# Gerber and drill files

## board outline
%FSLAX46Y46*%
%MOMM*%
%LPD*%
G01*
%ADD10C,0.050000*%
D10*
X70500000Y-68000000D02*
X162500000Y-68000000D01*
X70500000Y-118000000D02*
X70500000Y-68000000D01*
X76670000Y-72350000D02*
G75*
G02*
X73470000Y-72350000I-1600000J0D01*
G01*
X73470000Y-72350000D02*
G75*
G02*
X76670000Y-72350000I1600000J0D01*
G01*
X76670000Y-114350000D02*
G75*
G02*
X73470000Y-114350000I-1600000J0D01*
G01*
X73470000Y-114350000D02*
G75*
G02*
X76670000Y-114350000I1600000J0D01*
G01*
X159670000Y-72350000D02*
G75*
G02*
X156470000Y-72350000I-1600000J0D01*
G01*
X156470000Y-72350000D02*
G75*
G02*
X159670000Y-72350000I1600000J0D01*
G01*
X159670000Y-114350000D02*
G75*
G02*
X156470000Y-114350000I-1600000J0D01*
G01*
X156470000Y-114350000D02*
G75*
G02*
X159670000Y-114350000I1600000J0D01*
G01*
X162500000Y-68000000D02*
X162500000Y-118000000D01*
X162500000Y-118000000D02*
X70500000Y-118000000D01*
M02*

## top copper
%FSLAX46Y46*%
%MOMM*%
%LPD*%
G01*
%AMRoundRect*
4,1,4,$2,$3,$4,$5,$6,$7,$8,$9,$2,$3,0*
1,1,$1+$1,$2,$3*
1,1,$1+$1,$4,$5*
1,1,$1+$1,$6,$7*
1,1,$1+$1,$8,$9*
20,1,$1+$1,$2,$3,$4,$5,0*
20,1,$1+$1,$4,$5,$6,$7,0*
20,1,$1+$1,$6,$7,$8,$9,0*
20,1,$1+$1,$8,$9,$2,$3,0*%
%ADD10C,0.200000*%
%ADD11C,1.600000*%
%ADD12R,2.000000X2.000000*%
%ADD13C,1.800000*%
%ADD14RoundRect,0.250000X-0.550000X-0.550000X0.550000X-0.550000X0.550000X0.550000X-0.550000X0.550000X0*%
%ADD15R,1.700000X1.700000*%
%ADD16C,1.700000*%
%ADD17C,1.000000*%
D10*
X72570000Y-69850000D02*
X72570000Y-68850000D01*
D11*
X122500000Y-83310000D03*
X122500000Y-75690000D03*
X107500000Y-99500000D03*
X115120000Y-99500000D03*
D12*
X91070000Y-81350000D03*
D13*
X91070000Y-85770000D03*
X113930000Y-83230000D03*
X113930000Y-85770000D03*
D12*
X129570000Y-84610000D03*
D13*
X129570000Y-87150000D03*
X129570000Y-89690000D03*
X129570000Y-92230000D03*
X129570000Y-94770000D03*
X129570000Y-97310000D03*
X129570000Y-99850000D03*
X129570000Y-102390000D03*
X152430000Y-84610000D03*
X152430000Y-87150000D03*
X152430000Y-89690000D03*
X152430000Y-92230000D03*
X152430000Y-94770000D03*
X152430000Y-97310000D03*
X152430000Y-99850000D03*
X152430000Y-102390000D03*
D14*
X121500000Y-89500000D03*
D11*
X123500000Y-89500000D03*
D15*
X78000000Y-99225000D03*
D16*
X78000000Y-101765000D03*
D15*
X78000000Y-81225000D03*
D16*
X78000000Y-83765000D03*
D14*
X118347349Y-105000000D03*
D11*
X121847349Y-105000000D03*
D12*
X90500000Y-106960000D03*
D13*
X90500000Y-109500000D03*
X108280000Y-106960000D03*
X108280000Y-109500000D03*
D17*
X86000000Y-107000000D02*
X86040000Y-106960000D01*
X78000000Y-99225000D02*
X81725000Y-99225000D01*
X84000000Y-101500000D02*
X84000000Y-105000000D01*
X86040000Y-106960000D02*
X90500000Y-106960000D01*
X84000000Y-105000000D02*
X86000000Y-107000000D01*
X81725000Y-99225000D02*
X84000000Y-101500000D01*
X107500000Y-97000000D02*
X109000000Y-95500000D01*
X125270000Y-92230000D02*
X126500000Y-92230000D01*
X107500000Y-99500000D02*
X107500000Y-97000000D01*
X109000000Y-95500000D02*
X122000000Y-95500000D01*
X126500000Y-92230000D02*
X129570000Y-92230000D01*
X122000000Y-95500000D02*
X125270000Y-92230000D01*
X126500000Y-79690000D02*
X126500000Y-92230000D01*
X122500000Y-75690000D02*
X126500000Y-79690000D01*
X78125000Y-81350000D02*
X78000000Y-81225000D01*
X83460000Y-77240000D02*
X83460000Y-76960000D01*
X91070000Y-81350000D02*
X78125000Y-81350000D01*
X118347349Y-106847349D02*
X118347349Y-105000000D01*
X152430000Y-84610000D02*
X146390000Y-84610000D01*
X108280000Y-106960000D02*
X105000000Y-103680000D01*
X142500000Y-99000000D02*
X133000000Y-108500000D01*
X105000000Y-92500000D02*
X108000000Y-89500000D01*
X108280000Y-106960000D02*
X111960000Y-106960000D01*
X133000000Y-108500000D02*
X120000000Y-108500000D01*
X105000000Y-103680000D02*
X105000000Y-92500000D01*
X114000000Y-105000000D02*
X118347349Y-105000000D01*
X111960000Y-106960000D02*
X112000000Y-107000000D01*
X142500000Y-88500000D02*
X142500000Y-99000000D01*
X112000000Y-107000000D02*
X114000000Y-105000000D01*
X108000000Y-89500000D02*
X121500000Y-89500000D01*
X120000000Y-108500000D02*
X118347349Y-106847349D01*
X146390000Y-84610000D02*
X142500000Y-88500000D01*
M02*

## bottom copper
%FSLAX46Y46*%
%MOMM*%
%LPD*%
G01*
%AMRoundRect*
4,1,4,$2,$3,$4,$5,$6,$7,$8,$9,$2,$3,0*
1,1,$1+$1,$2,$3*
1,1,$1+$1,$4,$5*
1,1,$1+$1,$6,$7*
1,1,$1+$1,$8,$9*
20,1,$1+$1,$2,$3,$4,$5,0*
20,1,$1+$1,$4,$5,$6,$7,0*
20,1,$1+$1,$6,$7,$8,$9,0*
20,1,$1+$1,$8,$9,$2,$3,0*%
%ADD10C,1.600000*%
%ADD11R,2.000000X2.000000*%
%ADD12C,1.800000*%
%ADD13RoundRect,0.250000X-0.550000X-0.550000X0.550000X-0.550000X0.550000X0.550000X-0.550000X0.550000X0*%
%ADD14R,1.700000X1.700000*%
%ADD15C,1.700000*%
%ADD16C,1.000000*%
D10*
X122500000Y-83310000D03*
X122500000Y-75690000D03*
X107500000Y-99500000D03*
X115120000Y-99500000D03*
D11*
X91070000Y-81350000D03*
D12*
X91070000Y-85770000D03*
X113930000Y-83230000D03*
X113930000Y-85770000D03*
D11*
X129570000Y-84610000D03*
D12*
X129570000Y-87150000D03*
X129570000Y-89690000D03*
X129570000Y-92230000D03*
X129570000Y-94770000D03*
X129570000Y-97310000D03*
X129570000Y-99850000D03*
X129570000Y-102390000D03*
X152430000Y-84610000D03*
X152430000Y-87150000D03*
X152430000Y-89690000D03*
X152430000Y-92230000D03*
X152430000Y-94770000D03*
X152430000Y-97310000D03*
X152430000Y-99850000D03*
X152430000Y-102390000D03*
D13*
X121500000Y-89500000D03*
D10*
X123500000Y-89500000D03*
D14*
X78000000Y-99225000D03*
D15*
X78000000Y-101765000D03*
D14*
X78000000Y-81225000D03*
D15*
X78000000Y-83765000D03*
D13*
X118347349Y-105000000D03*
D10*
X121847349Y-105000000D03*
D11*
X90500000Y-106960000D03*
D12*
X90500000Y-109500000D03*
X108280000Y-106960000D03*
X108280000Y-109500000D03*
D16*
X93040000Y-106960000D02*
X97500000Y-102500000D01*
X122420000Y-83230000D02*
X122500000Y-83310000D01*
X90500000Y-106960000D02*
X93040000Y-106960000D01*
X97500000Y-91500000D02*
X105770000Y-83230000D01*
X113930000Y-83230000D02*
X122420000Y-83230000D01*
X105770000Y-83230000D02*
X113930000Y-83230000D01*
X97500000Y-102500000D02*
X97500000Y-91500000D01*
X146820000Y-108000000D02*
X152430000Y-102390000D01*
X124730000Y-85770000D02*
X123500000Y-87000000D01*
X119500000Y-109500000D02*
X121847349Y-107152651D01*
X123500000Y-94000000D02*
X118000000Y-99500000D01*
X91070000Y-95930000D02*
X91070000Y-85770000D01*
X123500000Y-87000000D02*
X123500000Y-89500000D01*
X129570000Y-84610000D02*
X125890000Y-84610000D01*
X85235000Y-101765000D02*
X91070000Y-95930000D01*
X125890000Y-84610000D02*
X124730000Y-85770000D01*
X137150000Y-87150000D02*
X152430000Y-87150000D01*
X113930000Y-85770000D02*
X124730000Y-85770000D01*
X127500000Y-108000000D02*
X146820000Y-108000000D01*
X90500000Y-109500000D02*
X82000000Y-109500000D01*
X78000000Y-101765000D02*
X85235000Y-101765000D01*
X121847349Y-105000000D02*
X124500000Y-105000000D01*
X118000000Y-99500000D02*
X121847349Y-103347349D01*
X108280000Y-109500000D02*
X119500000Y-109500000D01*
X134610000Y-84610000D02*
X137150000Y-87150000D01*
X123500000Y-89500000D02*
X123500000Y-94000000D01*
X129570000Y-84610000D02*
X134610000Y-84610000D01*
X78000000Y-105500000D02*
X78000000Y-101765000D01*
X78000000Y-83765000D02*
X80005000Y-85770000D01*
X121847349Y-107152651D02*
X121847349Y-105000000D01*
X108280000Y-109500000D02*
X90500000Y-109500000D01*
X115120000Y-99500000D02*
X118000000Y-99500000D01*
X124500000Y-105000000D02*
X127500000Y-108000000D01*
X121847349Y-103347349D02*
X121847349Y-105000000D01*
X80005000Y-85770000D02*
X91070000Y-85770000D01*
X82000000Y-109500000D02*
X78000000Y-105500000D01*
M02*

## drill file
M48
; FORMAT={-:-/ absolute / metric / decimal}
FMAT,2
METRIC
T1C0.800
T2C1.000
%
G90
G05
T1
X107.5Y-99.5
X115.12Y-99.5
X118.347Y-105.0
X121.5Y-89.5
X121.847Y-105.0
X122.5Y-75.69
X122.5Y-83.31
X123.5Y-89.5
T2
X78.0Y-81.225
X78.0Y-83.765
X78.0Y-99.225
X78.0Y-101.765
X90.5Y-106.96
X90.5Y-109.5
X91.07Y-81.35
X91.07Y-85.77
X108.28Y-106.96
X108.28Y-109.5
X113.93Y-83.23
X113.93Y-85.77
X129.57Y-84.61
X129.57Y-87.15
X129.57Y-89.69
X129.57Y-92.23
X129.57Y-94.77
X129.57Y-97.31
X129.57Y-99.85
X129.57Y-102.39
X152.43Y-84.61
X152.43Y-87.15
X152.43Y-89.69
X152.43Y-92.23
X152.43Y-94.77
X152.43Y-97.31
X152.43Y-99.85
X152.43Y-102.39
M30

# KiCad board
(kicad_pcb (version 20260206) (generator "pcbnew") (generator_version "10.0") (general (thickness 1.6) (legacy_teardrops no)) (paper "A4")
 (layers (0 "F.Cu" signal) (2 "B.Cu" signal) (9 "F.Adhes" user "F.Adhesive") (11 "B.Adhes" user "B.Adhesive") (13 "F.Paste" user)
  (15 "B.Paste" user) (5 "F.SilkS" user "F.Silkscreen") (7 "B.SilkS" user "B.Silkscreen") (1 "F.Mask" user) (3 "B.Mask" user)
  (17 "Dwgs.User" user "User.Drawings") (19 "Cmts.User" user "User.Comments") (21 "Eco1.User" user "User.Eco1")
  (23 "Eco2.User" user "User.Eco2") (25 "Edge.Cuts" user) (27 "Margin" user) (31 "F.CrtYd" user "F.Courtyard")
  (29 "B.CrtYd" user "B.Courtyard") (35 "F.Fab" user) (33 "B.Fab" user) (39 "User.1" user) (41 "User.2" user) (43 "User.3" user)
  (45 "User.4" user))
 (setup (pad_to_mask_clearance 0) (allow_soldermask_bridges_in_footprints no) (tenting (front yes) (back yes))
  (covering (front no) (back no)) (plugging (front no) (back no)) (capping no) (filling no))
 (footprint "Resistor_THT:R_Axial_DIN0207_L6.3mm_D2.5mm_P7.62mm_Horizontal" (layer "F.Cu") (at 122.5 83.31 90)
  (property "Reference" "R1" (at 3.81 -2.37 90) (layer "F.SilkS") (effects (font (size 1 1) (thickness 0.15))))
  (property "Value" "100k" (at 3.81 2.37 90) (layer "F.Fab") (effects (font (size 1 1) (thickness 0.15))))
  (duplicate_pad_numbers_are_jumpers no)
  (pad "1" thru_hole circle (at 0 0 90) (size 1.6 1.6) (drill 0.8) (layers "*.Cu" "*.Mask") (remove_unused_layers no) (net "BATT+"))
  (pad "2" thru_hole circle (at 7.62 0 90) (size 1.6 1.6) (drill 0.8) (layers "*.Cu" "*.Mask") (remove_unused_layers no) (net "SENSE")))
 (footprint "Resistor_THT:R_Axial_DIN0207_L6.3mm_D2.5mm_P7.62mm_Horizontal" (layer "F.Cu") (at 107.5 99.5)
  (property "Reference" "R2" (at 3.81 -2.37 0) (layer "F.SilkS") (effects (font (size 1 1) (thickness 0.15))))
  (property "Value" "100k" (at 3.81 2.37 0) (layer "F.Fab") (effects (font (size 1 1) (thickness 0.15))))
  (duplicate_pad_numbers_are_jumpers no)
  (pad "1" thru_hole circle (at 0 0) (size 1.6 1.6) (drill 0.8) (layers "*.Cu" "*.Mask") (remove_unused_layers no) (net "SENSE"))
  (pad "2" thru_hole circle (at 7.62 0) (size 1.6 1.6) (drill 0.8) (layers "*.Cu" "*.Mask") (remove_unused_layers no) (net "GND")))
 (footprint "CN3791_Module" (layer "F.Cu") (at 102.5 84.5)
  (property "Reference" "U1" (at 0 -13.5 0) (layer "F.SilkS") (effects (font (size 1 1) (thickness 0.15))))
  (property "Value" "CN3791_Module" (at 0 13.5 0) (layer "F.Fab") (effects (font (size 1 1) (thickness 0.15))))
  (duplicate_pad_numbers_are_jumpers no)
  (pad "1" thru_hole rect (at -11.43 -3.15) (size 2 2) (drill 1) (layers "*.Cu" "*.Mask") (remove_unused_layers no) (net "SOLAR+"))
  (pad "2" thru_hole circle (at -11.43 1.27) (size 1.8 1.8) (drill 1) (layers "*.Cu" "*.Mask") (remove_unused_layers no) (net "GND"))
  (pad "3" thru_hole circle (at 11.43 -1.27) (size 1.8 1.8) (drill 1) (layers "*.Cu" "*.Mask") (remove_unused_layers no) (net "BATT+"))
  (pad "4" thru_hole circle (at 11.43 1.27) (size 1.8 1.8) (drill 1) (layers "*.Cu" "*.Mask") (remove_unused_layers no) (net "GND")))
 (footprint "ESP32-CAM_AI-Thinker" (layer "F.Cu") (at 141 93.5)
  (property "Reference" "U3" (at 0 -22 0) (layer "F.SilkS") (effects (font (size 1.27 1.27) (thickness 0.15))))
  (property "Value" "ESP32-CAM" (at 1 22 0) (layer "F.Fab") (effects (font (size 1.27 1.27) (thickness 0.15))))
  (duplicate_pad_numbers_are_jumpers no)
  (pad "1" thru_hole rect (at -11.43 -8.89) (size 2 2) (drill 1) (layers "*.Cu" "*.Mask") (remove_unused_layers no) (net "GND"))
  (pad "2" thru_hole circle (at -11.43 -6.35) (size 1.8 1.8) (drill 1) (layers "*.Cu" "*.Mask") (remove_unused_layers no))
  (pad "3" thru_hole circle (at -11.43 -3.81) (size 1.8 1.8) (drill 1) (layers "*.Cu" "*.Mask") (remove_unused_layers no))
  (pad "4" thru_hole circle (at -11.43 -1.27) (size 1.8 1.8) (drill 1) (layers "*.Cu" "*.Mask") (remove_unused_layers no) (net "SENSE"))
  (pad "5" thru_hole circle (at -11.43 1.27) (size 1.8 1.8) (drill 1) (layers "*.Cu" "*.Mask") (remove_unused_layers no))
  (pad "6" thru_hole circle (at -11.43 3.81) (size 1.8 1.8) (drill 1) (layers "*.Cu" "*.Mask") (remove_unused_layers no))
  (pad "7" thru_hole circle (at -11.43 6.35) (size 1.8 1.8) (drill 1) (layers "*.Cu" "*.Mask") (remove_unused_layers no))
  (pad "8" thru_hole circle (at -11.43 8.89) (size 1.8 1.8) (drill 1) (layers "*.Cu" "*.Mask") (remove_unused_layers no))
  (pad "9" thru_hole circle (at 11.43 -8.89) (size 1.8 1.8) (drill 1) (layers "*.Cu" "*.Mask") (remove_unused_layers no) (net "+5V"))
  (pad "10" thru_hole circle (at 11.43 -6.35) (size 1.8 1.8) (drill 1) (layers "*.Cu" "*.Mask") (remove_unused_layers no) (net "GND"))
  (pad "11" thru_hole circle (at 11.43 -3.81) (size 1.8 1.8) (drill 1) (layers "*.Cu" "*.Mask") (remove_unused_layers no))
  (pad "12" thru_hole circle (at 11.43 -1.27) (size 1.8 1.8) (drill 1) (layers "*.Cu" "*.Mask") (remove_unused_layers no))
  (pad "13" thru_hole circle (at 11.43 1.27) (size 1.8 1.8) (drill 1) (layers "*.Cu" "*.Mask") (remove_unused_layers no))
  (pad "14" thru_hole circle (at 11.43 3.81) (size 1.8 1.8) (drill 1) (layers "*.Cu" "*.Mask") (remove_unused_layers no))
  (pad "15" thru_hole circle (at 11.43 6.35) (size 1.8 1.8) (drill 1) (layers "*.Cu" "*.Mask") (remove_unused_layers no))
  (pad "16" thru_hole circle (at 11.43 8.89) (size 1.8 1.8) (drill 1) (layers "*.Cu" "*.Mask") (remove_unused_layers no) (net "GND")))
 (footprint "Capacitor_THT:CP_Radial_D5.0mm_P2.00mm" (layer "F.Cu") (at 121.5 89.5)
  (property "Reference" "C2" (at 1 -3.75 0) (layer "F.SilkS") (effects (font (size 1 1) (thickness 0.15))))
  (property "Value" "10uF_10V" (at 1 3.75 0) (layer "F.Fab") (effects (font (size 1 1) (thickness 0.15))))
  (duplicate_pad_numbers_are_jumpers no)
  (pad "1" thru_hole roundrect (at 0 0) (size 1.6 1.6) (drill 0.8) (layers "*.Cu" "*.Mask") (remove_unused_layers no)
   (roundrect_rratio 0.15625) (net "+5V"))
  (pad "2" thru_hole circle (at 2 0) (size 1.6 1.6) (drill 0.8) (layers "*.Cu" "*.Mask") (remove_unused_layers no) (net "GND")))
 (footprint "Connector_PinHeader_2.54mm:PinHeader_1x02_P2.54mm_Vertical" (layer "F.Cu") (at 78 99.225)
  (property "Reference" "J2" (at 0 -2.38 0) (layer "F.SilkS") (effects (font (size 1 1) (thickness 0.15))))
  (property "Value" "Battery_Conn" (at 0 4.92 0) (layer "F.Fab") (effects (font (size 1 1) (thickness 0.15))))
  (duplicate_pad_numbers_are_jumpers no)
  (pad "1" thru_hole rect (at 0 0) (size 1.7 1.7) (drill 1) (layers "*.Cu" "*.Mask") (remove_unused_layers no) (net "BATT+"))
  (pad "2" thru_hole circle (at 0 2.54) (size 1.7 1.7) (drill 1) (layers "*.Cu" "*.Mask") (remove_unused_layers no) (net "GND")))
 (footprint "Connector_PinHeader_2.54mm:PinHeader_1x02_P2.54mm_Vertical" (layer "F.Cu") (at 78 81.225)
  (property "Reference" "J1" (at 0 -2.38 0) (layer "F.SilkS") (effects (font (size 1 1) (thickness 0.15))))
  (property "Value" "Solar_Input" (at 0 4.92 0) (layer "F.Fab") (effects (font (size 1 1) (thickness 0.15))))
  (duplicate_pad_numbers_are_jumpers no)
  (pad "1" thru_hole rect (at 0 0) (size 1.7 1.7) (drill 1) (layers "*.Cu" "*.Mask") (remove_unused_layers no) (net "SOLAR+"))
  (pad "2" thru_hole circle (at 0 2.54) (size 1.7 1.7) (drill 1) (layers "*.Cu" "*.Mask") (remove_unused_layers no) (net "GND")))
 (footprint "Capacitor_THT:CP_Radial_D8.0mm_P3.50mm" (layer "F.Cu") (at 118.347349 105)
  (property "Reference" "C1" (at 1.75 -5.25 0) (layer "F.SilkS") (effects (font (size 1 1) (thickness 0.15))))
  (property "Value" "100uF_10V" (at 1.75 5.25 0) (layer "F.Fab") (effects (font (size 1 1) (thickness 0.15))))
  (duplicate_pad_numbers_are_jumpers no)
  (pad "1" thru_hole roundrect (at 0 0) (size 1.6 1.6) (drill 0.8) (layers "*.Cu" "*.Mask") (remove_unused_layers no)
   (roundrect_rratio 0.15625) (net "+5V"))
  (pad "2" thru_hole circle (at 3.5 0) (size 1.6 1.6) (drill 0.8) (layers "*.Cu" "*.Mask") (remove_unused_layers no) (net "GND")))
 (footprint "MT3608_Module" (layer "F.Cu") (at 99.39 108.23)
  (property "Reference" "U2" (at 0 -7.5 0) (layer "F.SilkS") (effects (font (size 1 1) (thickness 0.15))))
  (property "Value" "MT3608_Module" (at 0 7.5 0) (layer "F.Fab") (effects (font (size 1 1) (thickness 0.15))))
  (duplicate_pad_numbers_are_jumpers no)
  (pad "1" thru_hole rect (at -8.89 -1.27) (size 2 2) (drill 1) (layers "*.Cu" "*.Mask") (remove_unused_layers no) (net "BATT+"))
  (pad "2" thru_hole circle (at -8.89 1.27) (size 1.8 1.8) (drill 1) (layers "*.Cu" "*.Mask") (remove_unused_layers no) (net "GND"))
  (pad "3" thru_hole circle (at 8.89 -1.27) (size 1.8 1.8) (drill 1) (layers "*.Cu" "*.Mask") (remove_unused_layers no) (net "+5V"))
  (pad "4" thru_hole circle (at 8.89 1.27) (size 1.8 1.8) (drill 1) (layers "*.Cu" "*.Mask") (remove_unused_layers no) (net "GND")))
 (gr_line (start 72.57 69.85) (end 72.57 68.85) (stroke (width 0.2) (type default)) (layer "F.Cu"))
 (gr_line (start 70.5 68) (end 162.5 68) (stroke (width 0.05) (type default)) (layer "Edge.Cuts"))
 (gr_line (start 70.5 118) (end 70.5 68) (stroke (width 0.05) (type default)) (layer "Edge.Cuts"))
 (gr_circle (center 75.07 72.35) (end 76.67 72.35) (stroke (width 0.05) (type solid)) (fill no) (layer "Edge.Cuts"))
 (gr_circle (center 75.07 114.35) (end 76.67 114.35) (stroke (width 0.05) (type solid)) (fill no) (layer "Edge.Cuts"))
 (gr_circle (center 158.07 72.35) (end 159.67 72.35) (stroke (width 0.05) (type solid)) (fill no) (layer "Edge.Cuts"))
 (gr_circle (center 158.07 114.35) (end 159.67 114.35) (stroke (width 0.05) (type solid)) (fill no) (layer "Edge.Cuts"))
 (gr_line (start 162.5 68) (end 162.5 118) (stroke (width 0.05) (type default)) (layer "Edge.Cuts"))
 (gr_line (start 162.5 118) (end 70.5 118) (stroke (width 0.05) (type default)) (layer "Edge.Cuts"))
 (segment (start 86 107) (end 86.04 106.96) (width 1) (layer "F.Cu") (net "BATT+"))
 (segment (start 78 99.225) (end 81.725 99.225) (width 1) (layer "F.Cu") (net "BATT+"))
 (segment (start 84 101.5) (end 84 105) (width 1) (layer "F.Cu") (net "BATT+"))
 (segment (start 86.04 106.96) (end 90.5 106.96) (width 1) (layer "F.Cu") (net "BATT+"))
 (segment (start 84 105) (end 86 107) (width 1) (layer "F.Cu") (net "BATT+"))
 (segment (start 81.725 99.225) (end 84 101.5) (width 1) (layer "F.Cu") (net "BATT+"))
 (segment (start 93.04 106.96) (end 97.5 102.5) (width 1) (layer "B.Cu") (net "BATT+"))
 (segment (start 122.42 83.23) (end 122.5 83.31) (width 1) (layer "B.Cu") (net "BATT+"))
 (segment (start 90.5 106.96) (end 93.04 106.96) (width 1) (layer "B.Cu") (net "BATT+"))
 (segment (start 97.5 91.5) (end 105.77 83.23) (width 1) (layer "B.Cu") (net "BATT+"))
 (segment (start 113.93 83.23) (end 122.42 83.23) (width 1) (layer "B.Cu") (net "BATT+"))
 (segment (start 105.77 83.23) (end 113.93 83.23) (width 1) (layer "B.Cu") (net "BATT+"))
 (segment (start 97.5 102.5) (end 97.5 91.5) (width 1) (layer "B.Cu") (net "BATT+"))
 (segment (start 107.5 97) (end 109 95.5) (width 1) (layer "F.Cu") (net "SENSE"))
 (segment (start 125.27 92.23) (end 126.5 92.23) (width 1) (layer "F.Cu") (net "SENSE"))
 (segment (start 107.5 99.5) (end 107.5 97) (width 1) (layer "F.Cu") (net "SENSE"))
 (segment (start 109 95.5) (end 122 95.5) (width 1) (layer "F.Cu") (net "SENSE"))
 (segment (start 126.5 92.23) (end 129.57 92.23) (width 1) (layer "F.Cu") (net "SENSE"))
 (segment (start 122 95.5) (end 125.27 92.23) (width 1) (layer "F.Cu") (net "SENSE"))
 (segment (start 126.5 79.69) (end 126.5 92.23) (width 1) (layer "F.Cu") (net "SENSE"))
 (segment (start 122.5 75.69) (end 126.5 79.69) (width 1) (layer "F.Cu") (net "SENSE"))
 (segment (start 146.82 108) (end 152.43 102.39) (width 1) (layer "B.Cu") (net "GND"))
 (segment (start 124.73 85.77) (end 123.5 87) (width 1) (layer "B.Cu") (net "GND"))
 (segment (start 119.5 109.5) (end 121.847349 107.152651) (width 1) (layer "B.Cu") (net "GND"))
 (segment (start 123.5 94) (end 118 99.5) (width 1) (layer "B.Cu") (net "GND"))
 (segment (start 91.07 95.93) (end 91.07 85.77) (width 1) (layer "B.Cu") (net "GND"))
 (segment (start 123.5 87) (end 123.5 89.5) (width 1) (layer "B.Cu") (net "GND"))
 (segment (start 129.57 84.61) (end 125.89 84.61) (width 1) (layer "B.Cu") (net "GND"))
 (segment (start 85.235 101.765) (end 91.07 95.93) (width 1) (layer "B.Cu") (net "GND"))
 (segment (start 125.89 84.61) (end 124.73 85.77) (width 1) (layer "B.Cu") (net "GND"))
 (segment (start 137.15 87.15) (end 152.43 87.15) (width 1) (layer "B.Cu") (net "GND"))
 (segment (start 113.93 85.77) (end 124.73 85.77) (width 1) (layer "B.Cu") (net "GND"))
 (segment (start 127.5 108) (end 146.82 108) (width 1) (layer "B.Cu") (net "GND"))
 (segment (start 90.5 109.5) (end 82 109.5) (width 1) (layer "B.Cu") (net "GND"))
 (segment (start 78 101.765) (end 85.235 101.765) (width 1) (layer "B.Cu") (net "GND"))
 (segment (start 121.847349 105) (end 124.5 105) (width 1) (layer "B.Cu") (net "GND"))
 (segment (start 118 99.5) (end 121.847349 103.347349) (width 1) (layer "B.Cu") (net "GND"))
 (segment (start 108.28 109.5) (end 119.5 109.5) (width 1) (layer "B.Cu") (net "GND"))
 (segment (start 134.61 84.61) (end 137.15 87.15) (width 1) (layer "B.Cu") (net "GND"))
 (segment (start 123.5 89.5) (end 123.5 94) (width 1) (layer "B.Cu") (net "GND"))
 (segment (start 129.57 84.61) (end 134.61 84.61) (width 1) (layer "B.Cu") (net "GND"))
 (segment (start 78 105.5) (end 78 101.765) (width 1) (layer "B.Cu") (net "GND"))
 (segment (start 78 83.765) (end 80.005 85.77) (width 1) (layer "B.Cu") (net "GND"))
 (segment (start 121.847349 107.152651) (end 121.847349 105) (width 1) (layer "B.Cu") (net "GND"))
 (segment (start 108.28 109.5) (end 90.5 109.5) (width 1) (layer "B.Cu") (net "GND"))
 (segment (start 115.12 99.5) (end 118 99.5) (width 1) (layer "B.Cu") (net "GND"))
 (segment (start 124.5 105) (end 127.5 108) (width 1) (layer "B.Cu") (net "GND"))
 (segment (start 121.847349 103.347349) (end 121.847349 105) (width 1) (layer "B.Cu") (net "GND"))
 (segment (start 80.005 85.77) (end 91.07 85.77) (width 1) (layer "B.Cu") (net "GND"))
 (segment (start 82 109.5) (end 78 105.5) (width 1) (layer "B.Cu") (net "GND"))
 (segment (start 78.125 81.35) (end 78 81.225) (width 1) (layer "F.Cu") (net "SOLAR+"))
 (segment (start 83.46 77.24) (end 83.46 76.96) (width 1) (layer "F.Cu") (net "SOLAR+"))
 (segment (start 91.07 81.35) (end 78.125 81.35) (width 1) (layer "F.Cu") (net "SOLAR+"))
 (segment (start 118.347349 106.847349) (end 118.347349 105) (width 1) (layer "F.Cu") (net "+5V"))
 (segment (start 152.43 84.61) (end 146.39 84.61) (width 1) (layer "F.Cu") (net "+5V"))
 (segment (start 108.28 106.96) (end 105 103.68) (width 1) (layer "F.Cu") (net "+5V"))
 (segment (start 142.5 99) (end 133 108.5) (width 1) (layer "F.Cu") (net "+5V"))
 (segment (start 105 92.5) (end 108 89.5) (width 1) (layer "F.Cu") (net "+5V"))
 (segment (start 108.28 106.96) (end 111.96 106.96) (width 1) (layer "F.Cu") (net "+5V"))
 (segment (start 133 108.5) (end 120 108.5) (width 1) (layer "F.Cu") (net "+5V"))
 (segment (start 105 103.68) (end 105 92.5) (width 1) (layer "F.Cu") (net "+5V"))
 (segment (start 114 105) (end 118.347349 105) (width 1) (layer "F.Cu") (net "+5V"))
 (segment (start 111.96 106.96) (end 112 107) (width 1) (layer "F.Cu") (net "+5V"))
 (segment (start 142.5 88.5) (end 142.5 99) (width 1) (layer "F.Cu") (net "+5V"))
 (segment (start 112 107) (end 114 105) (width 1) (layer "F.Cu") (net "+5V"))
 (segment (start 108 89.5) (end 121.5 89.5) (width 1) (layer "F.Cu") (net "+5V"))
 (segment (start 120 108.5) (end 118.347349 106.847349) (width 1) (layer "F.Cu") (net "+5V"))
 (segment (start 146.39 84.61) (end 142.5 88.5) (width 1) (layer "F.Cu") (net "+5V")))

